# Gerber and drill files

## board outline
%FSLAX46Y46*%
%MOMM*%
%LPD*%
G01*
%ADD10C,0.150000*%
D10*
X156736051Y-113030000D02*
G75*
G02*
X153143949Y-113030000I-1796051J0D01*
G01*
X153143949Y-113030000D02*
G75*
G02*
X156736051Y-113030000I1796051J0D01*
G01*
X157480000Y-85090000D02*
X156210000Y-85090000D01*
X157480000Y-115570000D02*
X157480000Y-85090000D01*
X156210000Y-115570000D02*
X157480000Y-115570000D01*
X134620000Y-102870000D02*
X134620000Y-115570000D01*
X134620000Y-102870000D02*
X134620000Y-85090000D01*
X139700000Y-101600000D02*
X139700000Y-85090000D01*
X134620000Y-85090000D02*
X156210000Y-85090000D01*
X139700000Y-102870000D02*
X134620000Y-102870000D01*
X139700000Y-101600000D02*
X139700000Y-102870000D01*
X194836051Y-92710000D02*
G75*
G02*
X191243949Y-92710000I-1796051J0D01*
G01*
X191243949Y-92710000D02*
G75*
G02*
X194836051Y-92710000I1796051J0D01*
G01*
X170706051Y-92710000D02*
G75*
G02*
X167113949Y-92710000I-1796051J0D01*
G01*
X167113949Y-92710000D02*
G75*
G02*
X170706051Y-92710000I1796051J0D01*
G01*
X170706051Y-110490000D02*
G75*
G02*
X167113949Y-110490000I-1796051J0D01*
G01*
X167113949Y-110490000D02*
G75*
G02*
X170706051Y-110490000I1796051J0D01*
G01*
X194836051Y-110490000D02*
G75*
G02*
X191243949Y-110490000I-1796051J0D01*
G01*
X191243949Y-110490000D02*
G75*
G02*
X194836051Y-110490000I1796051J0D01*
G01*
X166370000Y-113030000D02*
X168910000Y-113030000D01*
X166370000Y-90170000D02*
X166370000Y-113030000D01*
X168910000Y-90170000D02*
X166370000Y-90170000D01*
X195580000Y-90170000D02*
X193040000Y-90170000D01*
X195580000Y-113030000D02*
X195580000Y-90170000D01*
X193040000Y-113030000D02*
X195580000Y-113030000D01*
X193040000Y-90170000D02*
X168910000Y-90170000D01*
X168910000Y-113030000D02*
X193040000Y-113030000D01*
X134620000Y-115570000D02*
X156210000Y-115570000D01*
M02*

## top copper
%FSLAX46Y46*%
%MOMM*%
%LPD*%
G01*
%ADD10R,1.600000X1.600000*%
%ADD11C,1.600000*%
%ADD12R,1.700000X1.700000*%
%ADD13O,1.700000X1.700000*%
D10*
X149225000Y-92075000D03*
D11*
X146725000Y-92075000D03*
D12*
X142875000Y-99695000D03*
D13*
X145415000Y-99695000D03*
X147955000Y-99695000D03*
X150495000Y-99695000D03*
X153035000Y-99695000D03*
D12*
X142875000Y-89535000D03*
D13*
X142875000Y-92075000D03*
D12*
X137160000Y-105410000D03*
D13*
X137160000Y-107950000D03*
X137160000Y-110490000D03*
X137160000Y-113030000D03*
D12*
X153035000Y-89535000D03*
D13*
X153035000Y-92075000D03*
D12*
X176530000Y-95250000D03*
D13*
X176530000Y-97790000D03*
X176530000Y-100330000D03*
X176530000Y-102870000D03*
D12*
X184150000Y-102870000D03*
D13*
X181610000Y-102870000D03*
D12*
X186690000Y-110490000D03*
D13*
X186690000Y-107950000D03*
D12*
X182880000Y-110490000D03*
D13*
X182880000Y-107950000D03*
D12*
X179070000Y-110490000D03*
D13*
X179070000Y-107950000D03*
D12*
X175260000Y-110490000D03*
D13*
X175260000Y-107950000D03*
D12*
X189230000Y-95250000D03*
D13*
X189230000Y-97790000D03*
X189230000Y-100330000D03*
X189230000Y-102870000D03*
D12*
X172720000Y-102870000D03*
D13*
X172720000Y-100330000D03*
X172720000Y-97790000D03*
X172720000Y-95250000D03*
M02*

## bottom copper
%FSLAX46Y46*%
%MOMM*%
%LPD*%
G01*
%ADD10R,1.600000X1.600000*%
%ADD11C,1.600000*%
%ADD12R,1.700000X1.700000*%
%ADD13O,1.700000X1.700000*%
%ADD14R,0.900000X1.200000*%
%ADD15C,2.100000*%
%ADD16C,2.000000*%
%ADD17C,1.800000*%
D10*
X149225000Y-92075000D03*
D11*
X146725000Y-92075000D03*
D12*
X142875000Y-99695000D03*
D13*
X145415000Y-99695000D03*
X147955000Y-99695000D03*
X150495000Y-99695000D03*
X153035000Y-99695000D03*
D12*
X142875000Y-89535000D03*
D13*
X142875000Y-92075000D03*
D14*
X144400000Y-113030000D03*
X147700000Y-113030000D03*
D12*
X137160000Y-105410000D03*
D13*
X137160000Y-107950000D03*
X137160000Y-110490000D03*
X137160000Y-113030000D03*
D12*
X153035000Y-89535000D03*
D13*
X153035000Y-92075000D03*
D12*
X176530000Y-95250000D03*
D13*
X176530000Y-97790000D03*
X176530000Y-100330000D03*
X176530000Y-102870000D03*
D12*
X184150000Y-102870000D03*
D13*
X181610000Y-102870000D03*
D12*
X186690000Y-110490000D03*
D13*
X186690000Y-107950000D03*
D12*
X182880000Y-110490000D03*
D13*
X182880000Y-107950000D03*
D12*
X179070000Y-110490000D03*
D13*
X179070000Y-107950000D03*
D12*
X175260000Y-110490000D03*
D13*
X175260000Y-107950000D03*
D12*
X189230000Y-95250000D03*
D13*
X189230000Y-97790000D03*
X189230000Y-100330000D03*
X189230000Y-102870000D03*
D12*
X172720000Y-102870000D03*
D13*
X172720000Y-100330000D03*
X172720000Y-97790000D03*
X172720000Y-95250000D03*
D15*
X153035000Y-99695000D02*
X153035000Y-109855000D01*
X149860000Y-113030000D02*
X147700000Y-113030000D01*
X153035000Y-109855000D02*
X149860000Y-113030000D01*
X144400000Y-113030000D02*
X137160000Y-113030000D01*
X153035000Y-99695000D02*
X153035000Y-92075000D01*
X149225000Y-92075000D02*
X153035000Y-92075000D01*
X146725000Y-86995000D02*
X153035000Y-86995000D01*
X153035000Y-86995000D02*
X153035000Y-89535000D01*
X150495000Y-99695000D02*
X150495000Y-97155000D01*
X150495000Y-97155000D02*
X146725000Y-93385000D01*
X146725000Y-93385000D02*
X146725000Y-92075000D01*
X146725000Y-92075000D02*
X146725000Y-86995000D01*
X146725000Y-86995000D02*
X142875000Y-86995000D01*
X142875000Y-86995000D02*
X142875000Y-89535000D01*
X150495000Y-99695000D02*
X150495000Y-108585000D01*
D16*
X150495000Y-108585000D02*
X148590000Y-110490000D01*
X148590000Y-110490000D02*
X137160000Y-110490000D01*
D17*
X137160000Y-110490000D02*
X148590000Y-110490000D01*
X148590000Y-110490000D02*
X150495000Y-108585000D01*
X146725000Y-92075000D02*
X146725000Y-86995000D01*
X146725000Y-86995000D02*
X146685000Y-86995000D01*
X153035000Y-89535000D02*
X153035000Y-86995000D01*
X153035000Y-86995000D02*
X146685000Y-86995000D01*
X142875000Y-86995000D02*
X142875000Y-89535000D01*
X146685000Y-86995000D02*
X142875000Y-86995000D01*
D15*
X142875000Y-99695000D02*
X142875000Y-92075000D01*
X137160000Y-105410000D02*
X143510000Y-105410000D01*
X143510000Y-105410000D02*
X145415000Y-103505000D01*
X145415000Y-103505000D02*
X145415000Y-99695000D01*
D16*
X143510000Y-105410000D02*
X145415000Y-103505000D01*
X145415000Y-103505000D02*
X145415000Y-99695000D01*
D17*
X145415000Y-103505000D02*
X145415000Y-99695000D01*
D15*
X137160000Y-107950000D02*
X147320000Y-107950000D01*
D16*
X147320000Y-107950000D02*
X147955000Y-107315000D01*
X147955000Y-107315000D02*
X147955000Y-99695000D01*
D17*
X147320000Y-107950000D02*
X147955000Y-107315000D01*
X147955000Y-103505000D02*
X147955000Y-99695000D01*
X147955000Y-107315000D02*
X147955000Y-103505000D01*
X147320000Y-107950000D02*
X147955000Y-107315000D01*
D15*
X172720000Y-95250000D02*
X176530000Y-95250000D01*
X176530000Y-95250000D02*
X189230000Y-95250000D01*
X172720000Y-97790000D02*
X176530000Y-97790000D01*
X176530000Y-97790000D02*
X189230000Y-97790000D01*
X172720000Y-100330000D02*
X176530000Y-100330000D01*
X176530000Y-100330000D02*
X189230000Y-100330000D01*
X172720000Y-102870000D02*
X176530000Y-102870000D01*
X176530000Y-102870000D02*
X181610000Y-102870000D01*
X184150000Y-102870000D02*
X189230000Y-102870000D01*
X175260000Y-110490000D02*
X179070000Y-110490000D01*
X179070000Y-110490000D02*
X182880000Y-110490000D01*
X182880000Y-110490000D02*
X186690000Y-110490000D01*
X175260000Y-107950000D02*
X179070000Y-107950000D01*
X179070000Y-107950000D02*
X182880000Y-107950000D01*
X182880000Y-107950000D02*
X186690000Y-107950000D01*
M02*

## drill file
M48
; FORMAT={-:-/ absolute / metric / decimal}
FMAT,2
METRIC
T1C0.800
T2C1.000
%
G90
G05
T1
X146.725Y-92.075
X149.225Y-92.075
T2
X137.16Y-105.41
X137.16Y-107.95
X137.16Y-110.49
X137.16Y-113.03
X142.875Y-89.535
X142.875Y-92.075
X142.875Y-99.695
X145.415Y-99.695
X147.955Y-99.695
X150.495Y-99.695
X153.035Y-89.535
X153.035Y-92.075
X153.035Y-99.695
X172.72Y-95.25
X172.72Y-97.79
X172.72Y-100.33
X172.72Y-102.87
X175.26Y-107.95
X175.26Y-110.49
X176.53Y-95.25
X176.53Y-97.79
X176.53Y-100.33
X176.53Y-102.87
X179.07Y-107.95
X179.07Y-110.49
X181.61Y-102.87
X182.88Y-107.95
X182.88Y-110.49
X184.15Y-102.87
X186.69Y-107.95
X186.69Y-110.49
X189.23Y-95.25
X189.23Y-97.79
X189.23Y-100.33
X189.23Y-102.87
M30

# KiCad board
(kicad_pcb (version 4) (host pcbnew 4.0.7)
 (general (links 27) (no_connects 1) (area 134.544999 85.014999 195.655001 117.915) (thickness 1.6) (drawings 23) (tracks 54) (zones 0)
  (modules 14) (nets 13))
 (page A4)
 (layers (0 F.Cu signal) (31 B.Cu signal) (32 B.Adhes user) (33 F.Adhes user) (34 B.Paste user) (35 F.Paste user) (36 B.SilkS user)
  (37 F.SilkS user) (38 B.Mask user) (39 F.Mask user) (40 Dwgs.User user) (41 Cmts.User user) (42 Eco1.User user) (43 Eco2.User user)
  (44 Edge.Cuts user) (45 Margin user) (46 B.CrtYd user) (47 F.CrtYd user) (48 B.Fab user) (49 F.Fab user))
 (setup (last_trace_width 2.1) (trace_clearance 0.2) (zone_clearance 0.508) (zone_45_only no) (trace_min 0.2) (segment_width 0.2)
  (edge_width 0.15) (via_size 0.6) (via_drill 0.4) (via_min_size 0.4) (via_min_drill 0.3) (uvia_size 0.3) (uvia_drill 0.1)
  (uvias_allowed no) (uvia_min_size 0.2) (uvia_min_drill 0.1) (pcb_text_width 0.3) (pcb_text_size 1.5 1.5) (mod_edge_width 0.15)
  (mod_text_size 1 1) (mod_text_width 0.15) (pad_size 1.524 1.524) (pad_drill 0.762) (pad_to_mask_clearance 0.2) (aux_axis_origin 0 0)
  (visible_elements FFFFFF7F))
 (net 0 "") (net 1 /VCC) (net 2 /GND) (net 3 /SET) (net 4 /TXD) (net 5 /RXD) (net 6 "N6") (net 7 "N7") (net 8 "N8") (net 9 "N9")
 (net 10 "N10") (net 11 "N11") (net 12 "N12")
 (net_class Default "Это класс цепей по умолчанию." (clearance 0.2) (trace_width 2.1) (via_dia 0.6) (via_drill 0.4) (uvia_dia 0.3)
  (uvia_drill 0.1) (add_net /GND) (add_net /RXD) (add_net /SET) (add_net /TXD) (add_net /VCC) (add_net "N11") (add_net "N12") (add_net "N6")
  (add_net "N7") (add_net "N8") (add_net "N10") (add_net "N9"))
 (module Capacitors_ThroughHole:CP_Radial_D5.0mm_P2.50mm (layer F.Cu) (at 149.225 92.075 180)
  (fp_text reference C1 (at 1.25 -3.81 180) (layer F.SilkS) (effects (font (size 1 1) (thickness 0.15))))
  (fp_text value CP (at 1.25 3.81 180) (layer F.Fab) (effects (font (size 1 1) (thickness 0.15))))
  (pad 1 thru_hole rect (at 0 0 180) (size 1.6 1.6) (drill 0.8) (layers *.Cu *.Mask) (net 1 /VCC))
  (pad 2 thru_hole circle (at 2.5 0 180) (size 1.6 1.6) (drill 0.8) (layers *.Cu *.Mask) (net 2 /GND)))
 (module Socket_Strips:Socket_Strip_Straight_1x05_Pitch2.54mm (layer F.Cu) (at 142.875 99.695 90)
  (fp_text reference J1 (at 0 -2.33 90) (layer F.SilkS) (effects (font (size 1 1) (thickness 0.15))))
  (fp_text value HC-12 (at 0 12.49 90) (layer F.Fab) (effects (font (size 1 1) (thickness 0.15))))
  (pad 1 thru_hole rect (at 0 0 90) (size 1.7 1.7) (drill 1) (layers *.Cu *.Mask) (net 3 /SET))
  (pad 2 thru_hole oval (at 0 2.54 90) (size 1.7 1.7) (drill 1) (layers *.Cu *.Mask) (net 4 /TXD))
  (pad 3 thru_hole oval (at 0 5.08 90) (size 1.7 1.7) (drill 1) (layers *.Cu *.Mask) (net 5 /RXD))
  (pad 4 thru_hole oval (at 0 7.62 90) (size 1.7 1.7) (drill 1) (layers *.Cu *.Mask) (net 2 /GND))
  (pad 5 thru_hole oval (at 0 10.16 90) (size 1.7 1.7) (drill 1) (layers *.Cu *.Mask) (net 1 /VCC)))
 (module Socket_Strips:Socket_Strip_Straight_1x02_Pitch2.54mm (layer F.Cu) (at 142.875 89.535)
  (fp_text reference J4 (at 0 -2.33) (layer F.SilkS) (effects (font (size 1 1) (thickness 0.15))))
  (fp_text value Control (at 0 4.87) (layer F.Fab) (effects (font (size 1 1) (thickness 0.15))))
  (pad 1 thru_hole rect (at 0 0) (size 1.7 1.7) (drill 1) (layers *.Cu *.Mask) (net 2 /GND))
  (pad 2 thru_hole oval (at 0 2.54) (size 1.7 1.7) (drill 1) (layers *.Cu *.Mask) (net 3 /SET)))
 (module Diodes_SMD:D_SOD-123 (layer B.Cu) (at 146.05 113.03)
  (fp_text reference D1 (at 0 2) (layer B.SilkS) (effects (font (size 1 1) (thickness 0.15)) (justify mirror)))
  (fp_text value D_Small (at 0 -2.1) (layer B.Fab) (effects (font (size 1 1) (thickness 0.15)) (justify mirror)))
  (pad 1 smd rect (at -1.65 0) (size 0.9 1.2) (layers B.Cu B.Paste B.Mask) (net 1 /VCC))
  (pad 2 smd rect (at 1.65 0) (size 0.9 1.2) (layers B.Cu B.Paste B.Mask) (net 1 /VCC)))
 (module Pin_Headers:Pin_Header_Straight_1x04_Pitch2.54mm (layer F.Cu) (at 137.16 105.41)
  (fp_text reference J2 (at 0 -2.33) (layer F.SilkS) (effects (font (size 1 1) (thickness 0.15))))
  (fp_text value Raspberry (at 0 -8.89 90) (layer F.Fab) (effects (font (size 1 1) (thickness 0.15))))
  (pad 1 thru_hole rect (at 0 0) (size 1.7 1.7) (drill 1) (layers *.Cu *.Mask) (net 4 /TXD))
  (pad 2 thru_hole oval (at 0 2.54) (size 1.7 1.7) (drill 1) (layers *.Cu *.Mask) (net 5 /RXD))
  (pad 3 thru_hole oval (at 0 5.08) (size 1.7 1.7) (drill 1) (layers *.Cu *.Mask) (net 2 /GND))
  (pad 4 thru_hole oval (at 0 7.62) (size 1.7 1.7) (drill 1) (layers *.Cu *.Mask) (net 1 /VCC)))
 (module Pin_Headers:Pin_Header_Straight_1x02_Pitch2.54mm (layer F.Cu) (at 153.035 89.535)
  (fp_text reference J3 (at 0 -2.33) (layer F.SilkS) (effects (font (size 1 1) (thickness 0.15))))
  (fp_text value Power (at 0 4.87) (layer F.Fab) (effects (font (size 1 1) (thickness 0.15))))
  (pad 1 thru_hole rect (at 0 0) (size 1.7 1.7) (drill 1) (layers *.Cu *.Mask) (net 2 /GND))
  (pad 2 thru_hole oval (at 0 2.54) (size 1.7 1.7) (drill 1) (layers *.Cu *.Mask) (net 1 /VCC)))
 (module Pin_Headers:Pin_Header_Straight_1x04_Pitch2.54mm (layer F.Cu) (at 176.53 95.25)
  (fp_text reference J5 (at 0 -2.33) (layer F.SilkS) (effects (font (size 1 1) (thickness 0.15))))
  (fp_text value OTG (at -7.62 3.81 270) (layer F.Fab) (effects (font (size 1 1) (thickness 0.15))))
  (pad 1 thru_hole rect (at 0 0) (size 1.7 1.7) (drill 1) (layers *.Cu *.Mask) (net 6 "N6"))
  (pad 2 thru_hole oval (at 0 2.54) (size 1.7 1.7) (drill 1) (layers *.Cu *.Mask) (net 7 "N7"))
  (pad 3 thru_hole oval (at 0 5.08) (size 1.7 1.7) (drill 1) (layers *.Cu *.Mask) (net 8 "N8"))
  (pad 4 thru_hole oval (at 0 7.62) (size 1.7 1.7) (drill 1) (layers *.Cu *.Mask) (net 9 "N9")))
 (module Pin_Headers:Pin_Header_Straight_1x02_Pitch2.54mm (layer F.Cu) (at 184.15 102.87 270)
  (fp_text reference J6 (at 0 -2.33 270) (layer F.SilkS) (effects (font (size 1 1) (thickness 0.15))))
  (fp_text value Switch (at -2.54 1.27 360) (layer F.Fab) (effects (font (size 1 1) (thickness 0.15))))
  (pad 1 thru_hole rect (at 0 0 270) (size 1.7 1.7) (drill 1) (layers *.Cu *.Mask) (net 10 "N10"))
  (pad 2 thru_hole oval (at 0 2.54 270) (size 1.7 1.7) (drill 1) (layers *.Cu *.Mask) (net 9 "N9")))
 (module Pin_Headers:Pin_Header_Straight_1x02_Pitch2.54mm (layer F.Cu) (at 186.69 110.49 180)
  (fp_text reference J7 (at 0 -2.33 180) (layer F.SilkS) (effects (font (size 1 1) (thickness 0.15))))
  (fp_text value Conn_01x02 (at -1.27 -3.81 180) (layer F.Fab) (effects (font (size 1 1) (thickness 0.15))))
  (pad 1 thru_hole rect (at 0 0 180) (size 1.7 1.7) (drill 1) (layers *.Cu *.Mask) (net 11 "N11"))
  (pad 2 thru_hole oval (at 0 2.54 180) (size 1.7 1.7) (drill 1) (layers *.Cu *.Mask) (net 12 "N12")))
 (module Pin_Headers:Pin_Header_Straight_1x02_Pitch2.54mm (layer F.Cu) (at 182.88 110.49 180)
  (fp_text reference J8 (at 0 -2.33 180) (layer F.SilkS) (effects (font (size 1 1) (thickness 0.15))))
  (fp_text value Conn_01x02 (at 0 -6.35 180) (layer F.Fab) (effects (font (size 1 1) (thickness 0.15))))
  (pad 1 thru_hole rect (at 0 0 180) (size 1.7 1.7) (drill 1) (layers *.Cu *.Mask) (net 11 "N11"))
  (pad 2 thru_hole oval (at 0 2.54 180) (size 1.7 1.7) (drill 1) (layers *.Cu *.Mask) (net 12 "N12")))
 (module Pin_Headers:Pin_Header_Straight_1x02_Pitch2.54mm (layer F.Cu) (at 179.07 110.49 180)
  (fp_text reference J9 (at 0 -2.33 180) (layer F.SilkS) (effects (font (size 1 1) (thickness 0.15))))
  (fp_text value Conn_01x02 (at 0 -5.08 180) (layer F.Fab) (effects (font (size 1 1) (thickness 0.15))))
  (pad 1 thru_hole rect (at 0 0 180) (size 1.7 1.7) (drill 1) (layers *.Cu *.Mask) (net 11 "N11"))
  (pad 2 thru_hole oval (at 0 2.54 180) (size 1.7 1.7) (drill 1) (layers *.Cu *.Mask) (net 12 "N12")))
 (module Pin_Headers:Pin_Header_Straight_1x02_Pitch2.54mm (layer F.Cu) (at 175.26 110.49 180)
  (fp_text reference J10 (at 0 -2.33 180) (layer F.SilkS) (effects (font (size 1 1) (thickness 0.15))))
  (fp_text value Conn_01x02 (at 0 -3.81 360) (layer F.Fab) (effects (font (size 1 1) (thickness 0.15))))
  (pad 1 thru_hole rect (at 0 0 180) (size 1.7 1.7) (drill 1) (layers *.Cu *.Mask) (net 11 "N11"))
  (pad 2 thru_hole oval (at 0 2.54 180) (size 1.7 1.7) (drill 1) (layers *.Cu *.Mask) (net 12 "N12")))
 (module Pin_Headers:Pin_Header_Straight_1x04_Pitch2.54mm (layer F.Cu) (at 189.23 95.25)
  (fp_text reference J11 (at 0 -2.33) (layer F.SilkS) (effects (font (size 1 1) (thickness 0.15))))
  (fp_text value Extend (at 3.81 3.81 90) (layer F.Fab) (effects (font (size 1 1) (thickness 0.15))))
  (pad 1 thru_hole rect (at 0 0) (size 1.7 1.7) (drill 1) (layers *.Cu *.Mask) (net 6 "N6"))
  (pad 2 thru_hole oval (at 0 2.54) (size 1.7 1.7) (drill 1) (layers *.Cu *.Mask) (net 7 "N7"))
  (pad 3 thru_hole oval (at 0 5.08) (size 1.7 1.7) (drill 1) (layers *.Cu *.Mask) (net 8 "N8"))
  (pad 4 thru_hole oval (at 0 7.62) (size 1.7 1.7) (drill 1) (layers *.Cu *.Mask) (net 10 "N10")))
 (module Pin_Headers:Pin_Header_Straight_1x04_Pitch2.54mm (layer F.Cu) (at 172.72 102.87 180)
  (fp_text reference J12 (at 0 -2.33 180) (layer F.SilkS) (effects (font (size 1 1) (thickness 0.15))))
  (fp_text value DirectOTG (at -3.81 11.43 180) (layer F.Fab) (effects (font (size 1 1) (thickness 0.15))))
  (pad 1 thru_hole rect (at 0 0 180) (size 1.7 1.7) (drill 1) (layers *.Cu *.Mask) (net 9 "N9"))
  (pad 2 thru_hole oval (at 0 2.54 180) (size 1.7 1.7) (drill 1) (layers *.Cu *.Mask) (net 8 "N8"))
  (pad 3 thru_hole oval (at 0 5.08 180) (size 1.7 1.7) (drill 1) (layers *.Cu *.Mask) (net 7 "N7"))
  (pad 4 thru_hole oval (at 0 7.62 180) (size 1.7 1.7) (drill 1) (layers *.Cu *.Mask) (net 6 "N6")))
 (gr_circle (center 154.94 113.03) (end 156.21 114.3) (layer Edge.Cuts) (width 0.15))
 (gr_line (start 157.48 85.09) (end 156.21 85.09) (angle 90) (layer Edge.Cuts) (width 0.15))
 (gr_line (start 157.48 115.57) (end 157.48 85.09) (angle 90) (layer Edge.Cuts) (width 0.15))
 (gr_line (start 156.21 115.57) (end 157.48 115.57) (angle 90) (layer Edge.Cuts) (width 0.15))
 (gr_line (start 134.62 102.87) (end 134.62 115.57) (angle 90) (layer Edge.Cuts) (width 0.15))
 (gr_line (start 134.62 102.87) (end 134.62 85.09) (angle 90) (layer Edge.Cuts) (width 0.15))
 (gr_line (start 139.7 101.6) (end 139.7 85.09) (angle 90) (layer Edge.Cuts) (width 0.15))
 (gr_line (start 134.62 85.09) (end 156.21 85.09) (angle 90) (layer Edge.Cuts) (width 0.15))
 (gr_line (start 139.7 102.87) (end 134.62 102.87) (angle 90) (layer Edge.Cuts) (width 0.15))
 (gr_line (start 139.7 101.6) (end 139.7 102.87) (angle 90) (layer Edge.Cuts) (width 0.15))
 (gr_circle (center 193.04 92.71) (end 194.31 93.98) (layer Edge.Cuts) (width 0.15))
 (gr_circle (center 168.91 92.71) (end 170.18 93.98) (layer Edge.Cuts) (width 0.15))
 (gr_circle (center 168.91 110.49) (end 170.18 111.76) (layer Edge.Cuts) (width 0.15))
 (gr_circle (center 193.04 110.49) (end 194.31 111.76) (layer Edge.Cuts) (width 0.15))
 (gr_line (start 166.37 113.03) (end 168.91 113.03) (angle 90) (layer Edge.Cuts) (width 0.15))
 (gr_line (start 166.37 90.17) (end 166.37 113.03) (angle 90) (layer Edge.Cuts) (width 0.15))
 (gr_line (start 168.91 90.17) (end 166.37 90.17) (angle 90) (layer Edge.Cuts) (width 0.15))
 (gr_line (start 195.58 90.17) (end 193.04 90.17) (angle 90) (layer Edge.Cuts) (width 0.15))
 (gr_line (start 195.58 113.03) (end 195.58 90.17) (angle 90) (layer Edge.Cuts) (width 0.15))
 (gr_line (start 193.04 113.03) (end 195.58 113.03) (angle 90) (layer Edge.Cuts) (width 0.15))
 (gr_line (start 193.04 90.17) (end 168.91 90.17) (angle 90) (layer Edge.Cuts) (width 0.15))
 (gr_line (start 168.91 113.03) (end 193.04 113.03) (angle 90) (layer Edge.Cuts) (width 0.15))
 (gr_line (start 134.62 115.57) (end 156.21 115.57) (angle 90) (layer Edge.Cuts) (width 0.15))
 (segment (start 153.035 99.695) (end 153.035 109.855) (width 2.1) (layer B.Cu) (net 1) (status 400000))
 (segment (start 149.86 113.03) (end 147.7 113.03) (width 2.1) (layer B.Cu) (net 1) (status 800000))
 (segment (start 153.035 109.855) (end 149.86 113.03) (width 2.1) (layer B.Cu) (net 1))
 (segment (start 144.4 113.03) (end 137.16 113.03) (width 2.1) (layer B.Cu) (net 1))
 (segment (start 153.035 99.695) (end 153.035 92.075) (width 2.1) (layer B.Cu) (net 1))
 (segment (start 149.225 92.075) (end 153.035 92.075) (width 2.1) (layer B.Cu) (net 1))
 (segment (start 146.725 86.995) (end 153.035 86.995) (width 2.1) (layer B.Cu) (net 2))
 (segment (start 153.035 86.995) (end 153.035 89.535) (width 2.1) (layer B.Cu) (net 2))
 (segment (start 150.495 99.695) (end 150.495 97.155) (width 2.1) (layer B.Cu) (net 2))
 (segment (start 150.495 97.155) (end 146.725 93.385) (width 2.1) (layer B.Cu) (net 2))
 (segment (start 146.725 93.385) (end 146.725 92.075) (width 2.1) (layer B.Cu) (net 2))
 (segment (start 146.725 92.075) (end 146.725 86.995) (width 2.1) (layer B.Cu) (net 2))
 (segment (start 146.725 86.995) (end 142.875 86.995) (width 2.1) (layer B.Cu) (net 2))
 (segment (start 142.875 86.995) (end 142.875 89.535) (width 2.1) (layer B.Cu) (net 2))
 (segment (start 150.495 99.695) (end 150.495 108.585) (width 2.1) (layer B.Cu) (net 2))
 (segment (start 150.495 108.585) (end 148.59 110.49) (width 2) (layer B.Cu) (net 2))
 (segment (start 148.59 110.49) (end 137.16 110.49) (width 2) (layer B.Cu) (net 2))
 (segment (start 137.16 110.49) (end 148.59 110.49) (width 1.8) (layer B.Cu) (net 2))
 (segment (start 148.59 110.49) (end 150.495 108.585) (width 1.8) (layer B.Cu) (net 2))
 (segment (start 146.725 92.075) (end 146.725 86.995) (width 1.8) (layer B.Cu) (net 2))
 (segment (start 146.725 86.995) (end 146.685 86.995) (width 1.8) (layer B.Cu) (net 2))
 (segment (start 153.035 89.535) (end 153.035 86.995) (width 1.8) (layer B.Cu) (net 2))
 (segment (start 153.035 86.995) (end 146.685 86.995) (width 1.8) (layer B.Cu) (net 2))
 (segment (start 142.875 86.995) (end 142.875 89.535) (width 1.8) (layer B.Cu) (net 2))
 (segment (start 146.685 86.995) (end 142.875 86.995) (width 1.8) (layer B.Cu) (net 2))
 (segment (start 142.875 99.695) (end 142.875 92.075) (width 2.1) (layer B.Cu) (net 3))
 (segment (start 137.16 105.41) (end 143.51 105.41) (width 2.1) (layer B.Cu) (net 4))
 (segment (start 143.51 105.41) (end 145.415 103.505) (width 2.1) (layer B.Cu) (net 4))
 (segment (start 145.415 103.505) (end 145.415 99.695) (width 2.1) (layer B.Cu) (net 4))
 (segment (start 143.51 105.41) (end 145.415 103.505) (width 2) (layer B.Cu) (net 4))
 (segment (start 145.415 103.505) (end 145.415 99.695) (width 2) (layer B.Cu) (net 4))
 (segment (start 145.415 103.505) (end 145.415 99.695) (width 1.8) (layer B.Cu) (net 4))
 (segment (start 137.16 107.95) (end 147.32 107.95) (width 2.1) (layer B.Cu) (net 5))
 (segment (start 147.32 107.95) (end 147.955 107.315) (width 2) (layer B.Cu) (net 5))
 (segment (start 147.955 107.315) (end 147.955 99.695) (width 2) (layer B.Cu) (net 5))
 (segment (start 147.32 107.95) (end 147.955 107.315) (width 1.8) (layer B.Cu) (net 5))
 (segment (start 147.955 103.505) (end 147.955 99.695) (width 1.8) (layer B.Cu) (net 5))
 (segment (start 147.955 107.315) (end 147.955 103.505) (width 1.8) (layer B.Cu) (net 5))
 (segment (start 147.32 107.95) (end 147.955 107.315) (width 1.8) (layer B.Cu) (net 5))
 (segment (start 172.72 95.25) (end 176.53 95.25) (width 2.1) (layer B.Cu) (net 6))
 (segment (start 176.53 95.25) (end 189.23 95.25) (width 2.1) (layer B.Cu) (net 6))
 (segment (start 172.72 97.79) (end 176.53 97.79) (width 2.1) (layer B.Cu) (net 7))
 (segment (start 176.53 97.79) (end 189.23 97.79) (width 2.1) (layer B.Cu) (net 7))
 (segment (start 172.72 100.33) (end 176.53 100.33) (width 2.1) (layer B.Cu) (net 8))
 (segment (start 176.53 100.33) (end 189.23 100.33) (width 2.1) (layer B.Cu) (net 8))
 (segment (start 172.72 102.87) (end 176.53 102.87) (width 2.1) (layer B.Cu) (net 9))
 (segment (start 176.53 102.87) (end 181.61 102.87) (width 2.1) (layer B.Cu) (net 9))
 (segment (start 184.15 102.87) (end 189.23 102.87) (width 2.1) (layer B.Cu) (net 10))
 (segment (start 175.26 110.49) (end 179.07 110.49) (width 2.1) (layer B.Cu) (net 11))
 (segment (start 179.07 110.49) (end 182.88 110.49) (width 2.1) (layer B.Cu) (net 11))
 (segment (start 182.88 110.49) (end 186.69 110.49) (width 2.1) (layer B.Cu) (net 11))
 (segment (start 175.26 107.95) (end 179.07 107.95) (width 2.1) (layer B.Cu) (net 12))
 (segment (start 179.07 107.95) (end 182.88 107.95) (width 2.1) (layer B.Cu) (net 12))
 (segment (start 182.88 107.95) (end 186.69 107.95) (width 2.1) (layer B.Cu) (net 12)))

